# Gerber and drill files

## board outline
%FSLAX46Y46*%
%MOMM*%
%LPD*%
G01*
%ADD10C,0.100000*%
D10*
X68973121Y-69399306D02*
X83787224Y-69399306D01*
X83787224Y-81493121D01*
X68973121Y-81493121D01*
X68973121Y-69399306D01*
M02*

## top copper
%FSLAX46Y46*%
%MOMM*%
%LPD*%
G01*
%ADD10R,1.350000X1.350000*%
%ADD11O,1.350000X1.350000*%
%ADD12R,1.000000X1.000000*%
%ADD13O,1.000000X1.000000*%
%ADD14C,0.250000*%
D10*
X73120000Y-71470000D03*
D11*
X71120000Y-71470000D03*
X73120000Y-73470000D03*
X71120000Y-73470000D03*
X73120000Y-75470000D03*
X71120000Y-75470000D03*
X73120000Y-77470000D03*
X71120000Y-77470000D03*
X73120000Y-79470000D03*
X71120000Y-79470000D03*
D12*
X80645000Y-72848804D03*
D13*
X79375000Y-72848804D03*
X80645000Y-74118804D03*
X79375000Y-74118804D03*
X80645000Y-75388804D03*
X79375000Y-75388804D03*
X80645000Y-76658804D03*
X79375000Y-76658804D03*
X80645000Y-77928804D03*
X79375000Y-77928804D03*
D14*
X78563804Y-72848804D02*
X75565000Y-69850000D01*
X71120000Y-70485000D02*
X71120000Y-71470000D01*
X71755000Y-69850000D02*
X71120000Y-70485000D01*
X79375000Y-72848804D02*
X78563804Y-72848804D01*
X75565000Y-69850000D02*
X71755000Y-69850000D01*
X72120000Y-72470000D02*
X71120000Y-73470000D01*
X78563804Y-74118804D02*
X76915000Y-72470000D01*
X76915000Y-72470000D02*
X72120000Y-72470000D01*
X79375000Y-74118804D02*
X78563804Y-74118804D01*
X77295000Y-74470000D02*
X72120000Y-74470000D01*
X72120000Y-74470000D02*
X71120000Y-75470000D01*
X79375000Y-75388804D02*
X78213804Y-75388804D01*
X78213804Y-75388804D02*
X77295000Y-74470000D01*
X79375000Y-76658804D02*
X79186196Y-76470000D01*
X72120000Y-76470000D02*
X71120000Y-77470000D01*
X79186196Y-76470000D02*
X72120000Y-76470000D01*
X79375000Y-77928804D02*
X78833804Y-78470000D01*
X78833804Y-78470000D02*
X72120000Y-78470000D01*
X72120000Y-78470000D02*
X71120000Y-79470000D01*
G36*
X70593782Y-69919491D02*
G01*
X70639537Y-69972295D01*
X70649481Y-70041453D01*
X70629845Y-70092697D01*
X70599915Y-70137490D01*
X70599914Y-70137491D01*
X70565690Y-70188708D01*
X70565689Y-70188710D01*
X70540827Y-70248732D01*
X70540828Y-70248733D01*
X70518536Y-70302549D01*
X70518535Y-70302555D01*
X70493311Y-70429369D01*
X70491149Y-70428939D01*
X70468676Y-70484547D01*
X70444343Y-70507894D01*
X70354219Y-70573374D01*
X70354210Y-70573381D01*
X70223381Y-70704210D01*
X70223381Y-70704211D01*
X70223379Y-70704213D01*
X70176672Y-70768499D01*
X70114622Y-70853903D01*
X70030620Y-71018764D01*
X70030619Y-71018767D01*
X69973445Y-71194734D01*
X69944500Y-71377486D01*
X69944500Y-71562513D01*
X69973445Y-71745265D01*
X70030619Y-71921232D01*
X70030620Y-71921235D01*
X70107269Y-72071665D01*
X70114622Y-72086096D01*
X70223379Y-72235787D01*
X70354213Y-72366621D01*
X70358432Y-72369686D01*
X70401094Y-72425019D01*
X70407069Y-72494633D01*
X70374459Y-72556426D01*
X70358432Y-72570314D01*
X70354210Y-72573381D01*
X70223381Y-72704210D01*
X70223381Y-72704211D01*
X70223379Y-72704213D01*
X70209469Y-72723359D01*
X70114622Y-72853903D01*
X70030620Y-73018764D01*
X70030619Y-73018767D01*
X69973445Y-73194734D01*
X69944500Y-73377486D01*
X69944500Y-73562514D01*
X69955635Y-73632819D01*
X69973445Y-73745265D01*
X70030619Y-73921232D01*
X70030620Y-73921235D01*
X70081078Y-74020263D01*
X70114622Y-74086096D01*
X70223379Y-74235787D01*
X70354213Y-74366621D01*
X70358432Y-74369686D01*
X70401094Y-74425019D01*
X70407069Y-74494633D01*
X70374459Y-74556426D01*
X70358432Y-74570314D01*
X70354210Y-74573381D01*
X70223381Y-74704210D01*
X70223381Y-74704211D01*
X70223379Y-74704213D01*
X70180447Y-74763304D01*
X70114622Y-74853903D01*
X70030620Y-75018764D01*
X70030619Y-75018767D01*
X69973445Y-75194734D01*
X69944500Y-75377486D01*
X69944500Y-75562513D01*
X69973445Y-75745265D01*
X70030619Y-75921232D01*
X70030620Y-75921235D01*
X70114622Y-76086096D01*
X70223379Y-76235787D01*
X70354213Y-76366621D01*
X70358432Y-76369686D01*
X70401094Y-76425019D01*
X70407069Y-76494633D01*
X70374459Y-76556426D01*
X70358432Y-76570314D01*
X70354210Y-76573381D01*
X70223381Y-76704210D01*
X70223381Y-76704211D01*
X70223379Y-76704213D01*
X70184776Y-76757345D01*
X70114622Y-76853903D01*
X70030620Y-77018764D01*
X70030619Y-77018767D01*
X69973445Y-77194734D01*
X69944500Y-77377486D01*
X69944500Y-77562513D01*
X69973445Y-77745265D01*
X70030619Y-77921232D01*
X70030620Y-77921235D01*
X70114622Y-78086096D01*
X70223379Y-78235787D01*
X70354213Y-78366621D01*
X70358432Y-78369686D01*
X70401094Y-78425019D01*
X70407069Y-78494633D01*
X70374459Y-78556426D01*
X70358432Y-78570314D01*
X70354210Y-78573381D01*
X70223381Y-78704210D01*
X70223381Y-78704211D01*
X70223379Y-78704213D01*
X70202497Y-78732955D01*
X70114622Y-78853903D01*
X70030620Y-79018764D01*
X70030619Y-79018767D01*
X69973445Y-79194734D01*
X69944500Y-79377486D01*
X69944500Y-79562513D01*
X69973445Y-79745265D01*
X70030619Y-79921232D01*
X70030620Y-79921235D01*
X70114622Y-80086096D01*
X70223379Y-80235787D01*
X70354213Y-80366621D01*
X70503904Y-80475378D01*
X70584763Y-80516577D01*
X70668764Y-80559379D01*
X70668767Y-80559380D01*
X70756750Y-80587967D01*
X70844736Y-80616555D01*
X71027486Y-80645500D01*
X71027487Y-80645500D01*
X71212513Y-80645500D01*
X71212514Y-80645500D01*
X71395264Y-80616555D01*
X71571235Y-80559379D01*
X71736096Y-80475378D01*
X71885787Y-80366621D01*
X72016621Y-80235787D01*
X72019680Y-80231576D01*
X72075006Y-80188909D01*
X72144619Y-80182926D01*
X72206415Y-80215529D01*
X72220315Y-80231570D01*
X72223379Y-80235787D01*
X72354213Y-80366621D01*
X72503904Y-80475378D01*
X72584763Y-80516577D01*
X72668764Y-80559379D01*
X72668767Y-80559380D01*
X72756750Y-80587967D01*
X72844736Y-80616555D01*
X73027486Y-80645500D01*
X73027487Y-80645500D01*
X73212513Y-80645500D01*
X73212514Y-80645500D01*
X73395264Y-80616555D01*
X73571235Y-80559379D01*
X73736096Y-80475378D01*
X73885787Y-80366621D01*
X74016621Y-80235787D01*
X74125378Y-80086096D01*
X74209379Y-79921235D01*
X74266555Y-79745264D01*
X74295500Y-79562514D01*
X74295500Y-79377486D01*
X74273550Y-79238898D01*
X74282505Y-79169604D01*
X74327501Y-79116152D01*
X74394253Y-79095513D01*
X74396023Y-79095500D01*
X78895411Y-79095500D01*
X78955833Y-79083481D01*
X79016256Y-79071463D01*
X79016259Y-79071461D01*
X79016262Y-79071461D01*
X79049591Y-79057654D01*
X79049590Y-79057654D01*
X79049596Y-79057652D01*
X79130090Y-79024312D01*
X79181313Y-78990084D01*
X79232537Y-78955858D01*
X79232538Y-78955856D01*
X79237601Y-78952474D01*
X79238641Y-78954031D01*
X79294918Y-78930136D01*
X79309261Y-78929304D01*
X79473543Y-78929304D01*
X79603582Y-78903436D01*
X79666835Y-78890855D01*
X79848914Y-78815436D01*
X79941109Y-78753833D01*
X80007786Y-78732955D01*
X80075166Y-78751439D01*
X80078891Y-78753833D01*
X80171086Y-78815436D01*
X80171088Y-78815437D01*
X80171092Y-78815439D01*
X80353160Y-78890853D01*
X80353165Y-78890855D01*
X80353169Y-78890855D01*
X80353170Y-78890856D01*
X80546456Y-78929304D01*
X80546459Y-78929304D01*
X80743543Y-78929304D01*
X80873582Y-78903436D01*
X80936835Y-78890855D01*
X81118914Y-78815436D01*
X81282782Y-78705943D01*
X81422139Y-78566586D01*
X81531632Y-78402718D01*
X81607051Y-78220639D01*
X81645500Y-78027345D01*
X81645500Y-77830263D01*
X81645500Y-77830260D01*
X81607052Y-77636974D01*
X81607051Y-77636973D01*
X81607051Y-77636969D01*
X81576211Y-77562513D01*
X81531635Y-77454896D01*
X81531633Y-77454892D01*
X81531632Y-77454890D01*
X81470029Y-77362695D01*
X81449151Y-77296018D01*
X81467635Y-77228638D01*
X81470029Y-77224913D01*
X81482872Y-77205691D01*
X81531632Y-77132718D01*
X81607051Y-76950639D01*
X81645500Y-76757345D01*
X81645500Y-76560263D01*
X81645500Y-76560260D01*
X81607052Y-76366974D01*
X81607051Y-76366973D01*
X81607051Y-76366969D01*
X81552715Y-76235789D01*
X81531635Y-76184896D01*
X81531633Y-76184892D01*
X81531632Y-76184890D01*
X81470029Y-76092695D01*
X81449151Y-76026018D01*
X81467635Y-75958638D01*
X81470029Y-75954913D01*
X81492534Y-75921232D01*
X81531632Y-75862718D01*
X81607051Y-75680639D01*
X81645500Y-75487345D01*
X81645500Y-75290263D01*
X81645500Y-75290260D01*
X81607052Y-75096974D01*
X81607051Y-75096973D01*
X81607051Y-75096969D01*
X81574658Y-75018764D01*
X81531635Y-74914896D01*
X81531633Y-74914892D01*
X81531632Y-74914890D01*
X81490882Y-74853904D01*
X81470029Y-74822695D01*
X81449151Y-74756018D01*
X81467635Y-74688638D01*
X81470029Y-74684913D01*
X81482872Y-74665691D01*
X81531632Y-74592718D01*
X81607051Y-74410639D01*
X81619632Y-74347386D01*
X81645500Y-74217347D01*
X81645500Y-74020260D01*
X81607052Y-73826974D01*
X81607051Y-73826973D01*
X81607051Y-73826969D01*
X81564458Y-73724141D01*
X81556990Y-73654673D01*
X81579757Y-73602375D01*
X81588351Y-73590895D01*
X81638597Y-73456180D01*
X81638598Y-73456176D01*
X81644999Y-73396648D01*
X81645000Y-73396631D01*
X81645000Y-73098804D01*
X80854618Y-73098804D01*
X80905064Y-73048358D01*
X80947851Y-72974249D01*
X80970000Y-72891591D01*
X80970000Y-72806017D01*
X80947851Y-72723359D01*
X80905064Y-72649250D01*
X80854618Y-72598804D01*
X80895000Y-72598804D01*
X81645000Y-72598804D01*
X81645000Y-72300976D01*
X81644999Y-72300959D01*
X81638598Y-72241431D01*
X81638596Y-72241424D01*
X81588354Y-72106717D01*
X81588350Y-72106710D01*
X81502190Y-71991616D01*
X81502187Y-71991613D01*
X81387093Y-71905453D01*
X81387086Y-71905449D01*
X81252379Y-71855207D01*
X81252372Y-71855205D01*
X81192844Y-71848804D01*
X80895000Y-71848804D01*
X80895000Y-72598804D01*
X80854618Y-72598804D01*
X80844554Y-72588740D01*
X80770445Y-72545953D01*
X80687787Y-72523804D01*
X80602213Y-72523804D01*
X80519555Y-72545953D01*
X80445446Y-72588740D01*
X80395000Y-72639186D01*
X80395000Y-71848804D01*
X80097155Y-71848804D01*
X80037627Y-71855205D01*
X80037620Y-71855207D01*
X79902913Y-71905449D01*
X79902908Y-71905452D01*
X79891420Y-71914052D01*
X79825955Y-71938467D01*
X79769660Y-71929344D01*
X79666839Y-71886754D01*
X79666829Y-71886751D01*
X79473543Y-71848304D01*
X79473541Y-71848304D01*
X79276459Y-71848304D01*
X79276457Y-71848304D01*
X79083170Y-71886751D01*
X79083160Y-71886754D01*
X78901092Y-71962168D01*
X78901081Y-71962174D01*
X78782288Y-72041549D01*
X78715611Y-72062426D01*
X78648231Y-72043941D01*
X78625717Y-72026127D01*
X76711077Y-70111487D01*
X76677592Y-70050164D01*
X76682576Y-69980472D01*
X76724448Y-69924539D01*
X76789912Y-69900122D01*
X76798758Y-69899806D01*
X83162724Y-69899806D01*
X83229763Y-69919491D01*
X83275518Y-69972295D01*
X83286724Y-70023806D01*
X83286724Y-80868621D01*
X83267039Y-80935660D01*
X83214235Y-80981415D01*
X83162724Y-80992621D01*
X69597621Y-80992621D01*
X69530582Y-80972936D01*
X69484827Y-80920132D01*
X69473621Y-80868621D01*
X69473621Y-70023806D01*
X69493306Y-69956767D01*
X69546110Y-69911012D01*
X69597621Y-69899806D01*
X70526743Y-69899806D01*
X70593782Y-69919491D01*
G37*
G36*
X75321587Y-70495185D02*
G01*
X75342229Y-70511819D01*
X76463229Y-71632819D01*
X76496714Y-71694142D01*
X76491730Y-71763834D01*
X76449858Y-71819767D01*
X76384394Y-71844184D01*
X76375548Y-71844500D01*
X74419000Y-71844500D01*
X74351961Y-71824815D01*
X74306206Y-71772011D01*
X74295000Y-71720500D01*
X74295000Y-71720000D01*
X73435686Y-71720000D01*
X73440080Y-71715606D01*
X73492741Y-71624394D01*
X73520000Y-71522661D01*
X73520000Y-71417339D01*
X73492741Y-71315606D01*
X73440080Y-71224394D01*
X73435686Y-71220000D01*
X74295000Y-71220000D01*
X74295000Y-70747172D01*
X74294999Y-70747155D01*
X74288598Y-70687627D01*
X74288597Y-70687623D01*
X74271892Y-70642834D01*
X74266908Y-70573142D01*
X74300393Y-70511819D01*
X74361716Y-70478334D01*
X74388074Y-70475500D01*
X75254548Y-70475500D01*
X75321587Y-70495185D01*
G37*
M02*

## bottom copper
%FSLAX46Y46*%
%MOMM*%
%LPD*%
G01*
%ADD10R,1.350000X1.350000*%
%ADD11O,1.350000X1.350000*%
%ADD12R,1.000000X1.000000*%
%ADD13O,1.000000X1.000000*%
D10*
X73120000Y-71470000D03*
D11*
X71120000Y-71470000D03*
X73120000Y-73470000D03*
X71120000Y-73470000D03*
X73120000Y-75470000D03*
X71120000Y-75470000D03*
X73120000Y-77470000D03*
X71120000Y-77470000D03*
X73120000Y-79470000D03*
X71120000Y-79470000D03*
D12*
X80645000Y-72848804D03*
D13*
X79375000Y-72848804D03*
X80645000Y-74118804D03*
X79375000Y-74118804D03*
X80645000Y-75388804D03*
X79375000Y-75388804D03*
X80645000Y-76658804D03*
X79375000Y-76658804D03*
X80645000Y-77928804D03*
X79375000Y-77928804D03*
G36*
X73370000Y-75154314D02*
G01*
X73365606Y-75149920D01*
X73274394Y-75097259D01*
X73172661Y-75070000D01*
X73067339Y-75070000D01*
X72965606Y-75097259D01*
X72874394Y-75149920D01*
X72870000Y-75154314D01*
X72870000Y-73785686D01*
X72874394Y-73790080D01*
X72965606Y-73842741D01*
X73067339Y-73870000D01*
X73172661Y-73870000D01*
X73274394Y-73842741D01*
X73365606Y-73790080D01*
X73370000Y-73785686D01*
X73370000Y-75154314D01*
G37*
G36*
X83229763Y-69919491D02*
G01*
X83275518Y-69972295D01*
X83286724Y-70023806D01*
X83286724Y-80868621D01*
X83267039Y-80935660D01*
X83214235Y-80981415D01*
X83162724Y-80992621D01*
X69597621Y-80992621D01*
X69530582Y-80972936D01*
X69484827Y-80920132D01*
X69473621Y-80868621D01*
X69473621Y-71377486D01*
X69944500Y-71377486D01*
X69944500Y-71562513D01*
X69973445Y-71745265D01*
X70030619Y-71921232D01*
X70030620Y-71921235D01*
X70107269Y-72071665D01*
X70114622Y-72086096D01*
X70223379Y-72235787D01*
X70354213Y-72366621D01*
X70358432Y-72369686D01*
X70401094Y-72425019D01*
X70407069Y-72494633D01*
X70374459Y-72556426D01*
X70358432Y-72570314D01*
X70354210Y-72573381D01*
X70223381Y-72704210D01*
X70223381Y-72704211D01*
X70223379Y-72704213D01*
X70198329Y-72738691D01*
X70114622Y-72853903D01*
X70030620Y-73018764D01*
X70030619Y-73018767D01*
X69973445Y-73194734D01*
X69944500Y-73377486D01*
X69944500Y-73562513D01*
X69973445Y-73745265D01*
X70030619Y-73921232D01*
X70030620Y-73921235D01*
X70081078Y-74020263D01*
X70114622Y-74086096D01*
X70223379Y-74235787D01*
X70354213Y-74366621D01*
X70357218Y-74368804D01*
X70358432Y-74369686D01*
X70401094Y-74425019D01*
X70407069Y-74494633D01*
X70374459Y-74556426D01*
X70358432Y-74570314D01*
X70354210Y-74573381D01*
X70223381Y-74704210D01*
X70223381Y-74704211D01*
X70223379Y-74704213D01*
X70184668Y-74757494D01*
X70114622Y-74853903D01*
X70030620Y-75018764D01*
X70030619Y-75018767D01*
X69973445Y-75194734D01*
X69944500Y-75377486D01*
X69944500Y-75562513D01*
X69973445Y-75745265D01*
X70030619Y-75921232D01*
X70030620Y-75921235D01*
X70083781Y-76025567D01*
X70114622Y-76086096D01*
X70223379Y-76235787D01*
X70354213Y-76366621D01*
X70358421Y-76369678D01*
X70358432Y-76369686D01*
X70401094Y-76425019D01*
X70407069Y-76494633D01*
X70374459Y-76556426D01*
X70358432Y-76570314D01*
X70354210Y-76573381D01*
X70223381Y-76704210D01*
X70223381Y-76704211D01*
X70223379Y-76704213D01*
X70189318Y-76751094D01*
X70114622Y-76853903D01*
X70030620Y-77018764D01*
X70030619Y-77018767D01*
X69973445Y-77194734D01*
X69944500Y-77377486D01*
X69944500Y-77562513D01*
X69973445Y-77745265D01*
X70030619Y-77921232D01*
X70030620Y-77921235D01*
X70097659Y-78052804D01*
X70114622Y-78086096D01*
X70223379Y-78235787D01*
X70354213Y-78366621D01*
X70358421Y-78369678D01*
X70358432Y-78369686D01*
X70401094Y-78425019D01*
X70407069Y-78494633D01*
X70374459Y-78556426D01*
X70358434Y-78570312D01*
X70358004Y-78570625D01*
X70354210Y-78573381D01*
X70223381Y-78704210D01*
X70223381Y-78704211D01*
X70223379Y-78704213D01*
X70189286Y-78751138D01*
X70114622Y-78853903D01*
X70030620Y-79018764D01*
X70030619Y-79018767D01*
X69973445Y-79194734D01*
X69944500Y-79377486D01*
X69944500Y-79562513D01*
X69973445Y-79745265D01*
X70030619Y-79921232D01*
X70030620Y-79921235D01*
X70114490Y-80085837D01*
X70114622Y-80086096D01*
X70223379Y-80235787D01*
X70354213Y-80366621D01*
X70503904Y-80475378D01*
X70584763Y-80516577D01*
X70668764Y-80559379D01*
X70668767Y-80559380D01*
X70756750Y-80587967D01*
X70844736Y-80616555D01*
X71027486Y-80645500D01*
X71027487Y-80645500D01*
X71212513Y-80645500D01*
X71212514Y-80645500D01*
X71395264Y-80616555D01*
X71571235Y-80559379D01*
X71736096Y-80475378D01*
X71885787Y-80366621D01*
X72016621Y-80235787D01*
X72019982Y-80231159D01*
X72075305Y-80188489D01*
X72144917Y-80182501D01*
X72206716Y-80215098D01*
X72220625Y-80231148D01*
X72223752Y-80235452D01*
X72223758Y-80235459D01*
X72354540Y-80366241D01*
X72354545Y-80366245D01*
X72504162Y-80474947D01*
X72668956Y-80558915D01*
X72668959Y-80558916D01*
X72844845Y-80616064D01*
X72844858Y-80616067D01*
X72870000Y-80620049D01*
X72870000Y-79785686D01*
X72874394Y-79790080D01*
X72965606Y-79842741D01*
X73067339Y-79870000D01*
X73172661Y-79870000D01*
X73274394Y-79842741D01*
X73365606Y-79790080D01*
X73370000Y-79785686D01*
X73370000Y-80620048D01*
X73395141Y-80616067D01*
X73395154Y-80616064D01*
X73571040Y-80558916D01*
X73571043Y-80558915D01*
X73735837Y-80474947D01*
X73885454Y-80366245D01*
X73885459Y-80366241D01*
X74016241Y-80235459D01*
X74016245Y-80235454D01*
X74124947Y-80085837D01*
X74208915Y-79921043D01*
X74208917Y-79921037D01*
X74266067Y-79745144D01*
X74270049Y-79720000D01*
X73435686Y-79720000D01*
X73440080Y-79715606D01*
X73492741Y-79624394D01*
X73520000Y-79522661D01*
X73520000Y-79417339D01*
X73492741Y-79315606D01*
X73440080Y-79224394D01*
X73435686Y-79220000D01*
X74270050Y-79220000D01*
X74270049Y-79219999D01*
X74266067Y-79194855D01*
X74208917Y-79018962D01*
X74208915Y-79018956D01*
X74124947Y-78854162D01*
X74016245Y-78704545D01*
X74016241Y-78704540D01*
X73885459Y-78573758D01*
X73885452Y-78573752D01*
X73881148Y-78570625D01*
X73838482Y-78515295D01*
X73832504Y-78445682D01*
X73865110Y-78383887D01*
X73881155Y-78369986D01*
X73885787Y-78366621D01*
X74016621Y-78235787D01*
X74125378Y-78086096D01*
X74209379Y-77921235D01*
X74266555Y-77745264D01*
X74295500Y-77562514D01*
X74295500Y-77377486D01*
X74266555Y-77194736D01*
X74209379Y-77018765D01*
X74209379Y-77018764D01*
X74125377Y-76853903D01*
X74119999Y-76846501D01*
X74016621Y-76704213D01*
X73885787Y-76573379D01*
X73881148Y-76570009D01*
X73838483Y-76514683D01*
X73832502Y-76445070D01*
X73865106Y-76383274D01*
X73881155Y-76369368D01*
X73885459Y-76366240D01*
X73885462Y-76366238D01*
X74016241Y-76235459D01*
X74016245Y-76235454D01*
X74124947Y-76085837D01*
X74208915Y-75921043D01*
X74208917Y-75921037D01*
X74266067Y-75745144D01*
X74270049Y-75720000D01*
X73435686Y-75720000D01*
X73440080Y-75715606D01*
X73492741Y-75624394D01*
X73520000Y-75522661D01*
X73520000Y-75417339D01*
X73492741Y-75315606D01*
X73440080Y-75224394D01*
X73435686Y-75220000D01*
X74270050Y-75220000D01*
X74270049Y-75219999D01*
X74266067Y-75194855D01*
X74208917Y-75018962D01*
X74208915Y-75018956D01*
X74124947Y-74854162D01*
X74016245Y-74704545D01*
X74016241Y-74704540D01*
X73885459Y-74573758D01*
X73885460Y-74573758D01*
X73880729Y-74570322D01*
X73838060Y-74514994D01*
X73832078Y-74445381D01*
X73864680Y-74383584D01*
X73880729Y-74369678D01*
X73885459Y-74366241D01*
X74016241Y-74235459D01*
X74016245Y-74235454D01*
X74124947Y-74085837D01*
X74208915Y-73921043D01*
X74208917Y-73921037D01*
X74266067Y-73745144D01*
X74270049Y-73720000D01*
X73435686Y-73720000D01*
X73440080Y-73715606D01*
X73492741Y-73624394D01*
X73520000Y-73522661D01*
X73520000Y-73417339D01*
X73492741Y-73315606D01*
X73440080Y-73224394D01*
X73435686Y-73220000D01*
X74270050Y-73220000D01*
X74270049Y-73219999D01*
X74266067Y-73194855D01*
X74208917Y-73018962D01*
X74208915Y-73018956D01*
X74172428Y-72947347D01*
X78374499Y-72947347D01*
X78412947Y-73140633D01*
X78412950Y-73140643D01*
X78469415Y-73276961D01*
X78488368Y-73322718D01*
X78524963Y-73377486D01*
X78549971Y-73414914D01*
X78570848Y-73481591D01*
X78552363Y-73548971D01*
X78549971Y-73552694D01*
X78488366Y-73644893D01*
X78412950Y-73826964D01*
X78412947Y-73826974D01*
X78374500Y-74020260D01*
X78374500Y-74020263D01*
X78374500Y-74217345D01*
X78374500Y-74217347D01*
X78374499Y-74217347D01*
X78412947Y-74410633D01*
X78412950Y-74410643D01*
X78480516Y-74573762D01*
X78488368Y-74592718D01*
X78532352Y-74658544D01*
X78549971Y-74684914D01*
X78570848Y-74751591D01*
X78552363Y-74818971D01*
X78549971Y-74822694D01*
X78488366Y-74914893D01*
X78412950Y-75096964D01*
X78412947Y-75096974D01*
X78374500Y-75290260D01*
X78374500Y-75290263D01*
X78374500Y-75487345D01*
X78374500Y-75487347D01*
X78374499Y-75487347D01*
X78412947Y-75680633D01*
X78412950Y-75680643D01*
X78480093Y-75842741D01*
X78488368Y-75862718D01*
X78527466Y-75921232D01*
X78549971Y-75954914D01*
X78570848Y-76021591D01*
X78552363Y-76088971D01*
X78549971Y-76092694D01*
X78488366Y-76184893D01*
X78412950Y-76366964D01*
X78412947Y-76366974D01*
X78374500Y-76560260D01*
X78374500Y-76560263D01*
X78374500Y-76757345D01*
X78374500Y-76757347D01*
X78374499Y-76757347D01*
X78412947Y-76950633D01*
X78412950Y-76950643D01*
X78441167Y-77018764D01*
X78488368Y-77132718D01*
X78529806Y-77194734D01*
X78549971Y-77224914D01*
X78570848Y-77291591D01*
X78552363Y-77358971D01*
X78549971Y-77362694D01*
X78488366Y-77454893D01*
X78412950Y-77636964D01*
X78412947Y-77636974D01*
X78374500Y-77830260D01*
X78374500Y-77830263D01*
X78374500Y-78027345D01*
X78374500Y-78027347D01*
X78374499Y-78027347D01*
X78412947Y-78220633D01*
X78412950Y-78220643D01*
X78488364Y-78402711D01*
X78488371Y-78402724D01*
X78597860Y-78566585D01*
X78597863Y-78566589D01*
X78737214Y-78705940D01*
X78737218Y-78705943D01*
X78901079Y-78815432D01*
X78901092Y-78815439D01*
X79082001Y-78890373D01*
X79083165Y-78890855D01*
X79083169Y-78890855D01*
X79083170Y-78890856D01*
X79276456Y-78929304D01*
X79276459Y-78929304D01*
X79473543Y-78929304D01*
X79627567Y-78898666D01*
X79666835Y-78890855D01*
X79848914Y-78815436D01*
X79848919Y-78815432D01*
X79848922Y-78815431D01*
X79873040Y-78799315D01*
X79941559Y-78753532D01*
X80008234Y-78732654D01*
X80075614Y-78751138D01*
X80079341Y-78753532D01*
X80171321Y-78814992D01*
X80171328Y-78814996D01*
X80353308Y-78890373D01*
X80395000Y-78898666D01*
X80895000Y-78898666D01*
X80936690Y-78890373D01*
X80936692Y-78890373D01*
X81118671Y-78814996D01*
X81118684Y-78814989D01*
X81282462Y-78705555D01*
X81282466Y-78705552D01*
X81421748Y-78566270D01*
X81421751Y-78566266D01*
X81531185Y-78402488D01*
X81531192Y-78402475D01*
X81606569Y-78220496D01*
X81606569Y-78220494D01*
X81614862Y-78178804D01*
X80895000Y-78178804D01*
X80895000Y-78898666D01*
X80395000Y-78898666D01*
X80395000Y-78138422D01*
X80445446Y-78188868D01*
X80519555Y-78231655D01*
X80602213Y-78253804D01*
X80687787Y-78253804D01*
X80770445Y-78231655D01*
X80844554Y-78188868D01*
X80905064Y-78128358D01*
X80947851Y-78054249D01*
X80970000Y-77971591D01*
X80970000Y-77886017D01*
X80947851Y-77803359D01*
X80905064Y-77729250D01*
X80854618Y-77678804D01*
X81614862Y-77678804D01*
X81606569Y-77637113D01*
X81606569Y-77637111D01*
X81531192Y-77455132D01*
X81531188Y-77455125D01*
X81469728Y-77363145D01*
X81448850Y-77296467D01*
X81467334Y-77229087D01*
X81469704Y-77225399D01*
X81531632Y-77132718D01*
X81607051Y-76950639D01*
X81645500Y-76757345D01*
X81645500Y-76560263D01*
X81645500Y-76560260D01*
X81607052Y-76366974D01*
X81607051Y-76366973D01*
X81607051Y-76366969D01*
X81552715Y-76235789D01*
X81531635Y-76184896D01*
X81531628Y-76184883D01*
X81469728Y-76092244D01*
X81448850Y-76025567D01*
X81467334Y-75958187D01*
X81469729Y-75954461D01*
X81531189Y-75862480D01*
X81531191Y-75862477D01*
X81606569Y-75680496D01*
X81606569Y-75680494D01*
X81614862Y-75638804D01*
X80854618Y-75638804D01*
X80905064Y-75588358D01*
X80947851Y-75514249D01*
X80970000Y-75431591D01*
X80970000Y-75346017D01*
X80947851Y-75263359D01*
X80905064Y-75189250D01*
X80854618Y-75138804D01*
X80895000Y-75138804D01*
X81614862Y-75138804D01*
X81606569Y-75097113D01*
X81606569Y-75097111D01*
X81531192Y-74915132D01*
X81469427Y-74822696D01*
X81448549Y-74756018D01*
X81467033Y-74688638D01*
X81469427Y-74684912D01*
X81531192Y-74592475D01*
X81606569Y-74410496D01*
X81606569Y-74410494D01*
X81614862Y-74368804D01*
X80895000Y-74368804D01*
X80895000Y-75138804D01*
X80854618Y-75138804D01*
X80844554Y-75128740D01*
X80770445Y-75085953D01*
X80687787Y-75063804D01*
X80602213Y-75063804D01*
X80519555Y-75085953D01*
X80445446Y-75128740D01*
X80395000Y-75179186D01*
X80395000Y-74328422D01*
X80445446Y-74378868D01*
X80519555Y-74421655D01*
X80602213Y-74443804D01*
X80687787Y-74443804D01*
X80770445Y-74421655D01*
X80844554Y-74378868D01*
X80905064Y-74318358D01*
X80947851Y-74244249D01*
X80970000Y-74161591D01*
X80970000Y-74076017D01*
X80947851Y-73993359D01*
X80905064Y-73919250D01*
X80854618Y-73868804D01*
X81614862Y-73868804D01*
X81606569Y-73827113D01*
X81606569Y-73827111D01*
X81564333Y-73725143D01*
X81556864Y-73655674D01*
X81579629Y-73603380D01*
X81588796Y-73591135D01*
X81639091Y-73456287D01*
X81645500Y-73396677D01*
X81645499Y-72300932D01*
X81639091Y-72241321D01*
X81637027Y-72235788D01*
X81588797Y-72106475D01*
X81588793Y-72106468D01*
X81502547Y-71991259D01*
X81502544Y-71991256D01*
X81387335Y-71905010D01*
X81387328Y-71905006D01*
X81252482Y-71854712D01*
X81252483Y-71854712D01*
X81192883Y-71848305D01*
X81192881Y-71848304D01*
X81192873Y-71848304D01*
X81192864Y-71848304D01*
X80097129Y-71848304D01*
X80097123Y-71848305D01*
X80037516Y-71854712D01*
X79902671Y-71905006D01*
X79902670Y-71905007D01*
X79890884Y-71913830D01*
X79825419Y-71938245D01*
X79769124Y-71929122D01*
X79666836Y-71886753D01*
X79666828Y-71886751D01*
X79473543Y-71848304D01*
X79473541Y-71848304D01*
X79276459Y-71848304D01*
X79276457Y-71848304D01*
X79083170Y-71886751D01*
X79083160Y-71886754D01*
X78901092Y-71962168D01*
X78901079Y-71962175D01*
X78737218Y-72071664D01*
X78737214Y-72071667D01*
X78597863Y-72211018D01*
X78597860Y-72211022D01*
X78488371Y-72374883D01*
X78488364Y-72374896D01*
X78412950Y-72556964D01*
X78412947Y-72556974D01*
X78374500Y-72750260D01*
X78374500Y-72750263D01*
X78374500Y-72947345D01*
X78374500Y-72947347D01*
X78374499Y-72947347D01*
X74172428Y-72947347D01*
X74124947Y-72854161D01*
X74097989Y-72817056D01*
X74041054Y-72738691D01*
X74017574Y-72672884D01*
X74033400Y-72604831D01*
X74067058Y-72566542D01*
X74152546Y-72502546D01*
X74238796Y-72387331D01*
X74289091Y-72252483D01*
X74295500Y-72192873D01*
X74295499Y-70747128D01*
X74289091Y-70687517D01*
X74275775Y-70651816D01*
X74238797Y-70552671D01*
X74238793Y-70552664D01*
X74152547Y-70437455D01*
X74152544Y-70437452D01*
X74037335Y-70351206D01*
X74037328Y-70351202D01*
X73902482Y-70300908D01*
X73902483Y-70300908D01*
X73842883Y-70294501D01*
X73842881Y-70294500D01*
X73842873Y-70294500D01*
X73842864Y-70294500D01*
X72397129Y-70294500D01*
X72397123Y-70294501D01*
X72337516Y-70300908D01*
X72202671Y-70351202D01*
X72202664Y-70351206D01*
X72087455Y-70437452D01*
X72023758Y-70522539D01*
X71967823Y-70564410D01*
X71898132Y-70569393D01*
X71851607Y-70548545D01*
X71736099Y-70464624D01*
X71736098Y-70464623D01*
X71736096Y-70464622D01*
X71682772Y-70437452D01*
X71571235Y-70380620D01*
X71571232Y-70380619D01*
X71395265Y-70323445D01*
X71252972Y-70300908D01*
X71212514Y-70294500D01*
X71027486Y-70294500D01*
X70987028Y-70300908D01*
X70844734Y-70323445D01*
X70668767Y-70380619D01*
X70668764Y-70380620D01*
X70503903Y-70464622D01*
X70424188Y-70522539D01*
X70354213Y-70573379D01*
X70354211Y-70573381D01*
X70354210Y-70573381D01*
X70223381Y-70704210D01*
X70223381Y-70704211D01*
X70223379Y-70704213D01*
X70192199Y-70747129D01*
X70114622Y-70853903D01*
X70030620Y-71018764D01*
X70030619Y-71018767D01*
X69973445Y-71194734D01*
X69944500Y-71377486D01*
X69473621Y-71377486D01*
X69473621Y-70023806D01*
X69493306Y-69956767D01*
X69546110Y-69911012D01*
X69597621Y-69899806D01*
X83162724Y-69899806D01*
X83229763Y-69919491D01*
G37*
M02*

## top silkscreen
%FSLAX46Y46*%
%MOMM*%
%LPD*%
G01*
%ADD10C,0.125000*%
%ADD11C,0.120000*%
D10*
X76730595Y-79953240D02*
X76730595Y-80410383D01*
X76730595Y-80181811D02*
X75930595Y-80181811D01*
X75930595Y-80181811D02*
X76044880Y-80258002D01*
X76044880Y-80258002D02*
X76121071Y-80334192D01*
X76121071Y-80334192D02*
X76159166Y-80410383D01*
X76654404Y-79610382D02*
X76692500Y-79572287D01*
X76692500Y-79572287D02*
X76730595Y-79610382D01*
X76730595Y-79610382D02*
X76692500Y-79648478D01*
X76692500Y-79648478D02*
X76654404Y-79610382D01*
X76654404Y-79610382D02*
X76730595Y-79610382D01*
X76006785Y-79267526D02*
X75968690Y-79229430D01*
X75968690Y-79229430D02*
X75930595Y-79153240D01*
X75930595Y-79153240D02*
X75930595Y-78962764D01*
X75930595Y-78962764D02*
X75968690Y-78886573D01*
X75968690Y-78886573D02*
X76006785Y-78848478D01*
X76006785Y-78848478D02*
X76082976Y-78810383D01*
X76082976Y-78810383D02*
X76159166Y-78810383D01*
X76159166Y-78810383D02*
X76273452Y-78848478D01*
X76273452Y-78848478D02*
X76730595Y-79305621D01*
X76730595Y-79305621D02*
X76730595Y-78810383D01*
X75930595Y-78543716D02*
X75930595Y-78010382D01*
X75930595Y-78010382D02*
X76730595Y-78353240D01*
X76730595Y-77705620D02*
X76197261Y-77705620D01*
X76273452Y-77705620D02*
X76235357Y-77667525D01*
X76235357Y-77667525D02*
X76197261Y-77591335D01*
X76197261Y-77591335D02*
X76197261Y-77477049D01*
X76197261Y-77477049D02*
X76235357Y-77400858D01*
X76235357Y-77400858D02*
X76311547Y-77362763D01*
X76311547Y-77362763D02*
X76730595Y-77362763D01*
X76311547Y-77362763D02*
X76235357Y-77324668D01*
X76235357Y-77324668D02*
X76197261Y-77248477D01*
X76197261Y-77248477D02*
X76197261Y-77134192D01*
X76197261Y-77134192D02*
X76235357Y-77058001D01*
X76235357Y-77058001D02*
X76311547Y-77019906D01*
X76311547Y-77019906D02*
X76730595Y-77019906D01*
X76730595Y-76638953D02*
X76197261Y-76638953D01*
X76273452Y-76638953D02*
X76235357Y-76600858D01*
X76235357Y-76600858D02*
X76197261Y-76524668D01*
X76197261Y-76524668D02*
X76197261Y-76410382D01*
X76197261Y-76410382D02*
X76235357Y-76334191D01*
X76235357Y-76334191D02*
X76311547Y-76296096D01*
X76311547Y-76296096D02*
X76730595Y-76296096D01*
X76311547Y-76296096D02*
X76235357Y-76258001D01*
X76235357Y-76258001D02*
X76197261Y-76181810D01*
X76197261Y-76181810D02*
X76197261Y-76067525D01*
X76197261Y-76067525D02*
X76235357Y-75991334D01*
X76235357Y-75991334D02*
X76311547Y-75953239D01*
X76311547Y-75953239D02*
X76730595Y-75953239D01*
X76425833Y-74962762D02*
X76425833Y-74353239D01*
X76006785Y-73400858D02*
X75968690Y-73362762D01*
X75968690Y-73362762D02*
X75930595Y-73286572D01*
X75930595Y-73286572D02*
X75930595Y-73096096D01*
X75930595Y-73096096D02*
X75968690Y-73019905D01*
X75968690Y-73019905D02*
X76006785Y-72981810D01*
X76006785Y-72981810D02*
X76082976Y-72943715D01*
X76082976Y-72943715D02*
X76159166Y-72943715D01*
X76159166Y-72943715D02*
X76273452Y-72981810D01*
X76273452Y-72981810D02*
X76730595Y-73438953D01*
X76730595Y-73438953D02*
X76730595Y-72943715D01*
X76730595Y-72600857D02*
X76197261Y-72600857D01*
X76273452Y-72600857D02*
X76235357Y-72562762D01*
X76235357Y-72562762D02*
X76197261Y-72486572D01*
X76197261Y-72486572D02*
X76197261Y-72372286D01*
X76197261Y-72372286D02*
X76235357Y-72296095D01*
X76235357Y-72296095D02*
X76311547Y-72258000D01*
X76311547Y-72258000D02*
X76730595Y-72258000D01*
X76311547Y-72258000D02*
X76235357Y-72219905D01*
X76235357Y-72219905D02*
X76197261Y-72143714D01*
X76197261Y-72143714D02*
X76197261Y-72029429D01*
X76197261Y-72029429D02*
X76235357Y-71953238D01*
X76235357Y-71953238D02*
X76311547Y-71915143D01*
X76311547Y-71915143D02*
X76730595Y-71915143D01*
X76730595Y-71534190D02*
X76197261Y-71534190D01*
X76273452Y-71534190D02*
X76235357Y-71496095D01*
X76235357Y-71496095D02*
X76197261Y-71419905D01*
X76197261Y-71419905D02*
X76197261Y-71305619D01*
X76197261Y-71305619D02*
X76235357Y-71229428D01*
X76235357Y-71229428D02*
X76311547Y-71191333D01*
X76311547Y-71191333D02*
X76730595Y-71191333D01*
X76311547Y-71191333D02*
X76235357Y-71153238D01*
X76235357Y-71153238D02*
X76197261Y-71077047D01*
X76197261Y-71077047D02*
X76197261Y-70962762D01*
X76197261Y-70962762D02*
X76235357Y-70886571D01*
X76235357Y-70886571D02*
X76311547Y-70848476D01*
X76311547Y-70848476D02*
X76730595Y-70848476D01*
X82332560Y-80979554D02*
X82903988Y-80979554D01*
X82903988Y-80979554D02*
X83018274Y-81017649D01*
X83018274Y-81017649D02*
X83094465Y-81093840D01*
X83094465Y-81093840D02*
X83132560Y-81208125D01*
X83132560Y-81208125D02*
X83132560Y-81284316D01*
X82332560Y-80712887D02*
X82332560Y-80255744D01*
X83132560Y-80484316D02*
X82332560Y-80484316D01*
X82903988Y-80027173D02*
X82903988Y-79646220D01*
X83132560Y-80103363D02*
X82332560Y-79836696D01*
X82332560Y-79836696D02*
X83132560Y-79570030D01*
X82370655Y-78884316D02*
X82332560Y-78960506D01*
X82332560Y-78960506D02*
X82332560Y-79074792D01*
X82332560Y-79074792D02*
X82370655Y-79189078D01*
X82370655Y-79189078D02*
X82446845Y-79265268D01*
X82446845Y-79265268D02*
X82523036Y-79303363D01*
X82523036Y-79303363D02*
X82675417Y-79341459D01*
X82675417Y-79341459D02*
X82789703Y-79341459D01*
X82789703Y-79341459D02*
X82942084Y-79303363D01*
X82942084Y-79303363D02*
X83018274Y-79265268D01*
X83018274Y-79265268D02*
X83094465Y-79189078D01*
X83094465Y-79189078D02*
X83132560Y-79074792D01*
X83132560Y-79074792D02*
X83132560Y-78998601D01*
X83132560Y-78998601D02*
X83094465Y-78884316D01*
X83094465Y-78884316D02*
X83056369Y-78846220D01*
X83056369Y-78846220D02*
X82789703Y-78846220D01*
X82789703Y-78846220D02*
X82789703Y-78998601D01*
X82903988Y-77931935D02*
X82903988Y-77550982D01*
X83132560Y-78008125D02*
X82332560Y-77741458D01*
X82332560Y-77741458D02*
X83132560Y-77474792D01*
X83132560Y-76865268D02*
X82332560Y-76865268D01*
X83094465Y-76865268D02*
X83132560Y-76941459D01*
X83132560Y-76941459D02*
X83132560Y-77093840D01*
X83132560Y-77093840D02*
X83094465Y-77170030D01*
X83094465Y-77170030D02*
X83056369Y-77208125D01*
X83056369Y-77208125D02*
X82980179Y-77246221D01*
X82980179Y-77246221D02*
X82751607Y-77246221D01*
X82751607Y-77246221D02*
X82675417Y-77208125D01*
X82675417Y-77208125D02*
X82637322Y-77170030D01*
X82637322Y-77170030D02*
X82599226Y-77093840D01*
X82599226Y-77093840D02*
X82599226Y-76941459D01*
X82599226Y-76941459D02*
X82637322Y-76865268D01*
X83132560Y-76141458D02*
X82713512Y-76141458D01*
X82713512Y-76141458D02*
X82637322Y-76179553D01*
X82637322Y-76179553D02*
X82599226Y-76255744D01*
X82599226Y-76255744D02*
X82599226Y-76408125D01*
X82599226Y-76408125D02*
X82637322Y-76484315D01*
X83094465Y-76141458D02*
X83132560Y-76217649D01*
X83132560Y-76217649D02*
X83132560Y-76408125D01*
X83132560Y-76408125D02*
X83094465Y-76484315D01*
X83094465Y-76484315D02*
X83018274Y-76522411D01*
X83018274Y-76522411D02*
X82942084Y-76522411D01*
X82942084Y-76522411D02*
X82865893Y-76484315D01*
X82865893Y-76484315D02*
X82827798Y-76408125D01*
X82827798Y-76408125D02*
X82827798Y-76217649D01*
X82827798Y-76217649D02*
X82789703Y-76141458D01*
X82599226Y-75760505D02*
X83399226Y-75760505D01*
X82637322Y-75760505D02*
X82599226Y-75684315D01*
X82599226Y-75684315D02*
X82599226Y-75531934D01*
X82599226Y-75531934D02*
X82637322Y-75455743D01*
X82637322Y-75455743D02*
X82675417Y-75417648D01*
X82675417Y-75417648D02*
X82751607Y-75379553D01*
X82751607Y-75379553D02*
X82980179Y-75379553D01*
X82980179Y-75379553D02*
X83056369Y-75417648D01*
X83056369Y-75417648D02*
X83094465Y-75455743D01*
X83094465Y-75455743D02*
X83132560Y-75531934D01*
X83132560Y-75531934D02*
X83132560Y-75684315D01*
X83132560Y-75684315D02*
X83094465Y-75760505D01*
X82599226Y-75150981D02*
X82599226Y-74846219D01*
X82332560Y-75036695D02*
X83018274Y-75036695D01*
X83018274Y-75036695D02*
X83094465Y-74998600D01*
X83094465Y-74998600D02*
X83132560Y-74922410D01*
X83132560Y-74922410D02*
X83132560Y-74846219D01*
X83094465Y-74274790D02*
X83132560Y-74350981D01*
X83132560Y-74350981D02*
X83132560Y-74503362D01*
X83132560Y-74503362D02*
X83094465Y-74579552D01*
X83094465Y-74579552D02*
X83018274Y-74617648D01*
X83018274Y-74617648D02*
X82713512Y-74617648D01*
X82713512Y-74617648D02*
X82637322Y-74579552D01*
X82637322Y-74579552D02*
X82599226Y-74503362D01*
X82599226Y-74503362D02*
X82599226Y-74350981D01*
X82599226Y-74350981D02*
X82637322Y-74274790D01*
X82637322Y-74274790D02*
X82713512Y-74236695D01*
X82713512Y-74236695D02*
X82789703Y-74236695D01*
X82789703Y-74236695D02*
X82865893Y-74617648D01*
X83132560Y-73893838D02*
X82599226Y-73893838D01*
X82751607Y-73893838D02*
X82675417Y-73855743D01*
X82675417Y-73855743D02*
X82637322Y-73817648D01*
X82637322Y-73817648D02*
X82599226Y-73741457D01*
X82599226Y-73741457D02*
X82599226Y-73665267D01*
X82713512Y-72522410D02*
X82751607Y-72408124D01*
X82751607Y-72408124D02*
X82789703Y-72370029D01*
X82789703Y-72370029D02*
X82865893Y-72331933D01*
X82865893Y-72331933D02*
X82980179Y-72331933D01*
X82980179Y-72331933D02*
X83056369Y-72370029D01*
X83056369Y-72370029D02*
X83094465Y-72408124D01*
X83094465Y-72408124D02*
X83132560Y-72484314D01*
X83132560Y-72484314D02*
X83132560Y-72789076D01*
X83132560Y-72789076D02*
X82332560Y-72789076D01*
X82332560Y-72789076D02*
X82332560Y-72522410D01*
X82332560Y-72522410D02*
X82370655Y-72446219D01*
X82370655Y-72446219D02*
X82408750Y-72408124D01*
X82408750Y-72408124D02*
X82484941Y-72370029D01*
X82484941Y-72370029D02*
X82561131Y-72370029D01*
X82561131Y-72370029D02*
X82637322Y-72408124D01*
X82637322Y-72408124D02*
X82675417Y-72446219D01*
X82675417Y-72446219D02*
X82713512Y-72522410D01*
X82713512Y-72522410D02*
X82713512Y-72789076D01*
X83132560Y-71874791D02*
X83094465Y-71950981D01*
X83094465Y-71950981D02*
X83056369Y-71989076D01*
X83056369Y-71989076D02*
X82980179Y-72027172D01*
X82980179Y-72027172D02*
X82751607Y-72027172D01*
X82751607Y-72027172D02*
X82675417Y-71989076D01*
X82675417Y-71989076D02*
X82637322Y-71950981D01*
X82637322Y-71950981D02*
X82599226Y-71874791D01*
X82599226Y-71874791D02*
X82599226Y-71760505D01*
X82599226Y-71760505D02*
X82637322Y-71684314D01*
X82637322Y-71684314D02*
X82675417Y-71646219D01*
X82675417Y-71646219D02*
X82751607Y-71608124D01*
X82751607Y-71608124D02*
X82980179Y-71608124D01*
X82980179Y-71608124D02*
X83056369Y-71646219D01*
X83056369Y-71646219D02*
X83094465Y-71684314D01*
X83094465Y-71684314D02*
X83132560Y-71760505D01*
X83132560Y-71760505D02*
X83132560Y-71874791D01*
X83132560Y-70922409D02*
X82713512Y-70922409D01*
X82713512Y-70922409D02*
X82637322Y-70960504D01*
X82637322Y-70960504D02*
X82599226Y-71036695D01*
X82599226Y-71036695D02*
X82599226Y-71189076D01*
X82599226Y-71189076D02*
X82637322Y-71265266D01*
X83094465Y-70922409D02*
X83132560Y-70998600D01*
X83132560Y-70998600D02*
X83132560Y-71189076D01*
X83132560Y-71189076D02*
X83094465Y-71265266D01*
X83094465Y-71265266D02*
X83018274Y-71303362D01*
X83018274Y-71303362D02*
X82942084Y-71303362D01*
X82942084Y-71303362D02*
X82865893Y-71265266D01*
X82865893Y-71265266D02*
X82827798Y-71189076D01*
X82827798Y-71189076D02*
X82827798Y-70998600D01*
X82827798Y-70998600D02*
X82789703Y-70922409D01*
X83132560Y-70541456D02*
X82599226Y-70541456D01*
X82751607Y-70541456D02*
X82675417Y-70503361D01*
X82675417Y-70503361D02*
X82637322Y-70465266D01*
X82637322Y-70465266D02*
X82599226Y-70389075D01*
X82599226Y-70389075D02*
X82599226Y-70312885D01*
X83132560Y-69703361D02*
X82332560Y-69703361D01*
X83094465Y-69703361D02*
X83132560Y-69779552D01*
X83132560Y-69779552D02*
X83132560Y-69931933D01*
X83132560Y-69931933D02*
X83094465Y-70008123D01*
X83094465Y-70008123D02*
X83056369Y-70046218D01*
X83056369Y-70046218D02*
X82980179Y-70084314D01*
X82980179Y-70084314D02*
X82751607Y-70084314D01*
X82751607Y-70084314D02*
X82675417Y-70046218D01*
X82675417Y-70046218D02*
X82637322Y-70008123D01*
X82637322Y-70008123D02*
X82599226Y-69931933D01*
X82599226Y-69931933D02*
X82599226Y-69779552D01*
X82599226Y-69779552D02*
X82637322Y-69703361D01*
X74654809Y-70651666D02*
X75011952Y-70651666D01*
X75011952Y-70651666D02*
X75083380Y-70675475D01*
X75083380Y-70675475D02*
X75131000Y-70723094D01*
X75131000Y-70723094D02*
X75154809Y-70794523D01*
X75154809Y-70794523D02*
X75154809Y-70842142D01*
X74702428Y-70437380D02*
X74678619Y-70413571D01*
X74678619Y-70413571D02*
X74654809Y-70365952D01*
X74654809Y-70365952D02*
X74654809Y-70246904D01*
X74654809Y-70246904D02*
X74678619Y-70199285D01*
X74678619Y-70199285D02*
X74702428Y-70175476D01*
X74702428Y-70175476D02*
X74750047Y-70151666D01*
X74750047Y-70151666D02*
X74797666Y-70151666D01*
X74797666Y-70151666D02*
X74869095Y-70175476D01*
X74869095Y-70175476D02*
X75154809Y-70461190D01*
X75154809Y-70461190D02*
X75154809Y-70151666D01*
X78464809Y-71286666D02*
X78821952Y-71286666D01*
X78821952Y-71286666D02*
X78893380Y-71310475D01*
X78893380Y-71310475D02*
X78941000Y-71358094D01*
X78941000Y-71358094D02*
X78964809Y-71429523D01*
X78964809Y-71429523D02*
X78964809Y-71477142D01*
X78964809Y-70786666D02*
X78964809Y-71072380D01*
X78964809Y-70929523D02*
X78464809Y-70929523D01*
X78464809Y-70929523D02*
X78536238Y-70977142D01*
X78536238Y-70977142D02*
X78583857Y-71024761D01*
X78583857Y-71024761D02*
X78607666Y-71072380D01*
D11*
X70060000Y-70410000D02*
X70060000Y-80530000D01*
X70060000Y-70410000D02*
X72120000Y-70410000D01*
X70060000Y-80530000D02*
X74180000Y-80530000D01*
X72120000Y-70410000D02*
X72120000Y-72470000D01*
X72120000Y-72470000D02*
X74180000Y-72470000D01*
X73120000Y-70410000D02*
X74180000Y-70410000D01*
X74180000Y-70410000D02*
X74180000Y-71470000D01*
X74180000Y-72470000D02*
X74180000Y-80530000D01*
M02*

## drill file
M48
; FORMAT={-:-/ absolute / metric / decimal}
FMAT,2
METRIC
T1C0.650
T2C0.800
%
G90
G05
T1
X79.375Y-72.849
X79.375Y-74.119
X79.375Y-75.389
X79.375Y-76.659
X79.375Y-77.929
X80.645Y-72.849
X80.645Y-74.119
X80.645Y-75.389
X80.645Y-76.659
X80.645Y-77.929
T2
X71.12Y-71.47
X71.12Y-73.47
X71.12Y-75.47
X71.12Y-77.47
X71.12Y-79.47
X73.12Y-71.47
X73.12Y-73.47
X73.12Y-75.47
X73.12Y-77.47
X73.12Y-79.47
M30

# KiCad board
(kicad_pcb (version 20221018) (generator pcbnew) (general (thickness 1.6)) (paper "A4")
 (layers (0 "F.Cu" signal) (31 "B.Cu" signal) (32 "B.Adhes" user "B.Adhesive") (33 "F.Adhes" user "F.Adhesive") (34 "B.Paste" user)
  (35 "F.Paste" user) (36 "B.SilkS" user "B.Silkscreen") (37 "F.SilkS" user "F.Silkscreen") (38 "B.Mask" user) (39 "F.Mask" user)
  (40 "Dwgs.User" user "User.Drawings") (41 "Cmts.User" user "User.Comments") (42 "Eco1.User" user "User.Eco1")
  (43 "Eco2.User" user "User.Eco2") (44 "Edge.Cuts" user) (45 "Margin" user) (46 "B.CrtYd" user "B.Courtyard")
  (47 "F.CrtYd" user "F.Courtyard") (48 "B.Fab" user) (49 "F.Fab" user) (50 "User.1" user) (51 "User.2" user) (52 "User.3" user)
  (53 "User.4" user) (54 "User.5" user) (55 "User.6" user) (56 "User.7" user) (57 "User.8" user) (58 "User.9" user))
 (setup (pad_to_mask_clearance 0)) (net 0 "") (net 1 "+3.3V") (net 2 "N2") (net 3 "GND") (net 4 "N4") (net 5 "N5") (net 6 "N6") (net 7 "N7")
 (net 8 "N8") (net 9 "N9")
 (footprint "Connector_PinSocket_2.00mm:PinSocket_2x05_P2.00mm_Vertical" (layer "F.Cu") (at 73.12 71.47)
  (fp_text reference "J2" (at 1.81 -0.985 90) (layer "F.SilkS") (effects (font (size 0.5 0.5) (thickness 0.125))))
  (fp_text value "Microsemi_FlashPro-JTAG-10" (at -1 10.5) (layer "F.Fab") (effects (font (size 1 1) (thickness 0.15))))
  (fp_line (start -3.06 -1.06) (end -3.06 9.06) (stroke (width 0.12) (type solid)) (layer "F.SilkS"))
  (fp_line (start -3.06 -1.06) (end -1 -1.06) (stroke (width 0.12) (type solid)) (layer "F.SilkS"))
  (fp_line (start -3.06 9.06) (end 1.06 9.06) (stroke (width 0.12) (type solid)) (layer "F.SilkS"))
  (fp_line (start -1 -1.06) (end -1 1) (stroke (width 0.12) (type solid)) (layer "F.SilkS"))
  (fp_line (start -1 1) (end 1.06 1) (stroke (width 0.12) (type solid)) (layer "F.SilkS"))
  (fp_line (start 0 -1.06) (end 1.06 -1.06) (stroke (width 0.12) (type solid)) (layer "F.SilkS"))
  (fp_line (start 1.06 -1.06) (end 1.06 0) (stroke (width 0.12) (type solid)) (layer "F.SilkS"))
  (fp_line (start 1.06 1) (end 1.06 9.06) (stroke (width 0.12) (type solid)) (layer "F.SilkS"))
  (pad "1" thru_hole rect (at 0 0) (size 1.35 1.35) (drill 0.8) (layers "*.Cu" "*.Mask") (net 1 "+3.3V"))
  (pad "2" thru_hole oval (at -2 0) (size 1.35 1.35) (drill 0.8) (layers "*.Cu" "*.Mask") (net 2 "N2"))
  (pad "3" thru_hole oval (at 0 2) (size 1.35 1.35) (drill 0.8) (layers "*.Cu" "*.Mask") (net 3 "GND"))
  (pad "4" thru_hole oval (at -2 2) (size 1.35 1.35) (drill 0.8) (layers "*.Cu" "*.Mask") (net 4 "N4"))
  (pad "5" thru_hole oval (at 0 4) (size 1.35 1.35) (drill 0.8) (layers "*.Cu" "*.Mask") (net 3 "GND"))
  (pad "6" thru_hole oval (at -2 4) (size 1.35 1.35) (drill 0.8) (layers "*.Cu" "*.Mask") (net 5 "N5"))
  (pad "7" thru_hole oval (at 0 6) (size 1.35 1.35) (drill 0.8) (layers "*.Cu" "*.Mask") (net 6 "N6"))
  (pad "8" thru_hole oval (at -2 6) (size 1.35 1.35) (drill 0.8) (layers "*.Cu" "*.Mask") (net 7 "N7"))
  (pad "9" thru_hole oval (at 0 8) (size 1.35 1.35) (drill 0.8) (layers "*.Cu" "*.Mask") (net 3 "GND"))
  (pad "10" thru_hole oval (at -2 8) (size 1.35 1.35) (drill 0.8) (layers "*.Cu" "*.Mask") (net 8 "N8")))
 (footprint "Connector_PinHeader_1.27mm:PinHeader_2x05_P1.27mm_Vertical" (layer "B.Cu") (at 80.645 72.848804 180)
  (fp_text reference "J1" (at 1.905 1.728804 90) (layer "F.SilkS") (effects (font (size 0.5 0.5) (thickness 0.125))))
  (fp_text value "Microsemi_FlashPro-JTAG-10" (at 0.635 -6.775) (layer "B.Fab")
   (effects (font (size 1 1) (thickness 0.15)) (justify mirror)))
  (pad "1" thru_hole rect (at 0 0 180) (size 1 1) (drill 0.65) (layers "*.Cu" "*.Mask") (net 1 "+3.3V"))
  (pad "2" thru_hole oval (at 1.27 0 180) (size 1 1) (drill 0.65) (layers "*.Cu" "*.Mask") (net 2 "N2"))
  (pad "3" thru_hole oval (at 0 -1.27 180) (size 1 1) (drill 0.65) (layers "*.Cu" "*.Mask") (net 3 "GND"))
  (pad "4" thru_hole oval (at 1.27 -1.27 180) (size 1 1) (drill 0.65) (layers "*.Cu" "*.Mask") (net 4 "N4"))
  (pad "5" thru_hole oval (at 0 -2.54 180) (size 1 1) (drill 0.65) (layers "*.Cu" "*.Mask") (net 3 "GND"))
  (pad "6" thru_hole oval (at 1.27 -2.54 180) (size 1 1) (drill 0.65) (layers "*.Cu" "*.Mask") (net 5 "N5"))
  (pad "7" thru_hole oval (at 0 -3.81 180) (size 1 1) (drill 0.65) (layers "*.Cu" "*.Mask") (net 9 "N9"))
  (pad "8" thru_hole oval (at 1.27 -3.81 180) (size 1 1) (drill 0.65) (layers "*.Cu" "*.Mask") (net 7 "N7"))
  (pad "9" thru_hole oval (at 0 -5.08 180) (size 1 1) (drill 0.65) (layers "*.Cu" "*.Mask") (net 3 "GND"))
  (pad "10" thru_hole oval (at 1.27 -5.08 180) (size 1 1) (drill 0.65) (layers "*.Cu" "*.Mask") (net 8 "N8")))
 (gr_rect (start 68.973121 69.399306) (end 83.787224 81.493121) (stroke (width 0.1) (type default)) (fill none) (layer "Edge.Cuts"))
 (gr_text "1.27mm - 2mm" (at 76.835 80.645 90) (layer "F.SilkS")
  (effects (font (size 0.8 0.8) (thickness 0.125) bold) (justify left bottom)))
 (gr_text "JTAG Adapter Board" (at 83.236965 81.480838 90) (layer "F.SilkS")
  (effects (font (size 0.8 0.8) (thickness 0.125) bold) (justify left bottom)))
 (segment (start 78.563804 72.848804) (end 75.565 69.85) (width 0.25) (layer "F.Cu") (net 2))
 (segment (start 71.12 70.485) (end 71.12 71.47) (width 0.25) (layer "F.Cu") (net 2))
 (segment (start 71.755 69.85) (end 71.12 70.485) (width 0.25) (layer "F.Cu") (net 2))
 (segment (start 79.375 72.848804) (end 78.563804 72.848804) (width 0.25) (layer "F.Cu") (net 2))
 (segment (start 75.565 69.85) (end 71.755 69.85) (width 0.25) (layer "F.Cu") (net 2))
 (segment (start 72.12 72.47) (end 71.12 73.47) (width 0.25) (layer "F.Cu") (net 4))
 (segment (start 78.563804 74.118804) (end 76.915 72.47) (width 0.25) (layer "F.Cu") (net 4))
 (segment (start 76.915 72.47) (end 72.12 72.47) (width 0.25) (layer "F.Cu") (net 4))
 (segment (start 79.375 74.118804) (end 78.563804 74.118804) (width 0.25) (layer "F.Cu") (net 4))
 (segment (start 77.295 74.47) (end 72.12 74.47) (width 0.25) (layer "F.Cu") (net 5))
 (segment (start 72.12 74.47) (end 71.12 75.47) (width 0.25) (layer "F.Cu") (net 5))
 (segment (start 79.375 75.388804) (end 78.213804 75.388804) (width 0.25) (layer "F.Cu") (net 5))
 (segment (start 78.213804 75.388804) (end 77.295 74.47) (width 0.25) (layer "F.Cu") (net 5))
 (segment (start 79.375 76.658804) (end 79.186196 76.47) (width 0.25) (layer "F.Cu") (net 7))
 (segment (start 72.12 76.47) (end 71.12 77.47) (width 0.25) (layer "F.Cu") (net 7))
 (segment (start 79.186196 76.47) (end 72.12 76.47) (width 0.25) (layer "F.Cu") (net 7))
 (segment (start 79.375 77.928804) (end 78.833804 78.47) (width 0.25) (layer "F.Cu") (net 8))
 (segment (start 78.833804 78.47) (end 72.12 78.47) (width 0.25) (layer "F.Cu") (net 8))
 (segment (start 72.12 78.47) (end 71.12 79.47) (width 0.25) (layer "F.Cu") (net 8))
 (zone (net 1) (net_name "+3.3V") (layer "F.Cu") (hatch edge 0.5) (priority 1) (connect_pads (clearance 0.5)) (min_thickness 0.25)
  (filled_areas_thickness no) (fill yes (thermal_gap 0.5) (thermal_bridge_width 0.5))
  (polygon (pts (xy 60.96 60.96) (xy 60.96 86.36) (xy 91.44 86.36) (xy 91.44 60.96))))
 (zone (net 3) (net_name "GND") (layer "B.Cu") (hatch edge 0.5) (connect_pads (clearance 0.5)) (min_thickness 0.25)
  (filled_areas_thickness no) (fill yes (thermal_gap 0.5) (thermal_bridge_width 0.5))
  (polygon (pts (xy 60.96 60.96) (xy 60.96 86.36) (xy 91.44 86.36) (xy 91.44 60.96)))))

